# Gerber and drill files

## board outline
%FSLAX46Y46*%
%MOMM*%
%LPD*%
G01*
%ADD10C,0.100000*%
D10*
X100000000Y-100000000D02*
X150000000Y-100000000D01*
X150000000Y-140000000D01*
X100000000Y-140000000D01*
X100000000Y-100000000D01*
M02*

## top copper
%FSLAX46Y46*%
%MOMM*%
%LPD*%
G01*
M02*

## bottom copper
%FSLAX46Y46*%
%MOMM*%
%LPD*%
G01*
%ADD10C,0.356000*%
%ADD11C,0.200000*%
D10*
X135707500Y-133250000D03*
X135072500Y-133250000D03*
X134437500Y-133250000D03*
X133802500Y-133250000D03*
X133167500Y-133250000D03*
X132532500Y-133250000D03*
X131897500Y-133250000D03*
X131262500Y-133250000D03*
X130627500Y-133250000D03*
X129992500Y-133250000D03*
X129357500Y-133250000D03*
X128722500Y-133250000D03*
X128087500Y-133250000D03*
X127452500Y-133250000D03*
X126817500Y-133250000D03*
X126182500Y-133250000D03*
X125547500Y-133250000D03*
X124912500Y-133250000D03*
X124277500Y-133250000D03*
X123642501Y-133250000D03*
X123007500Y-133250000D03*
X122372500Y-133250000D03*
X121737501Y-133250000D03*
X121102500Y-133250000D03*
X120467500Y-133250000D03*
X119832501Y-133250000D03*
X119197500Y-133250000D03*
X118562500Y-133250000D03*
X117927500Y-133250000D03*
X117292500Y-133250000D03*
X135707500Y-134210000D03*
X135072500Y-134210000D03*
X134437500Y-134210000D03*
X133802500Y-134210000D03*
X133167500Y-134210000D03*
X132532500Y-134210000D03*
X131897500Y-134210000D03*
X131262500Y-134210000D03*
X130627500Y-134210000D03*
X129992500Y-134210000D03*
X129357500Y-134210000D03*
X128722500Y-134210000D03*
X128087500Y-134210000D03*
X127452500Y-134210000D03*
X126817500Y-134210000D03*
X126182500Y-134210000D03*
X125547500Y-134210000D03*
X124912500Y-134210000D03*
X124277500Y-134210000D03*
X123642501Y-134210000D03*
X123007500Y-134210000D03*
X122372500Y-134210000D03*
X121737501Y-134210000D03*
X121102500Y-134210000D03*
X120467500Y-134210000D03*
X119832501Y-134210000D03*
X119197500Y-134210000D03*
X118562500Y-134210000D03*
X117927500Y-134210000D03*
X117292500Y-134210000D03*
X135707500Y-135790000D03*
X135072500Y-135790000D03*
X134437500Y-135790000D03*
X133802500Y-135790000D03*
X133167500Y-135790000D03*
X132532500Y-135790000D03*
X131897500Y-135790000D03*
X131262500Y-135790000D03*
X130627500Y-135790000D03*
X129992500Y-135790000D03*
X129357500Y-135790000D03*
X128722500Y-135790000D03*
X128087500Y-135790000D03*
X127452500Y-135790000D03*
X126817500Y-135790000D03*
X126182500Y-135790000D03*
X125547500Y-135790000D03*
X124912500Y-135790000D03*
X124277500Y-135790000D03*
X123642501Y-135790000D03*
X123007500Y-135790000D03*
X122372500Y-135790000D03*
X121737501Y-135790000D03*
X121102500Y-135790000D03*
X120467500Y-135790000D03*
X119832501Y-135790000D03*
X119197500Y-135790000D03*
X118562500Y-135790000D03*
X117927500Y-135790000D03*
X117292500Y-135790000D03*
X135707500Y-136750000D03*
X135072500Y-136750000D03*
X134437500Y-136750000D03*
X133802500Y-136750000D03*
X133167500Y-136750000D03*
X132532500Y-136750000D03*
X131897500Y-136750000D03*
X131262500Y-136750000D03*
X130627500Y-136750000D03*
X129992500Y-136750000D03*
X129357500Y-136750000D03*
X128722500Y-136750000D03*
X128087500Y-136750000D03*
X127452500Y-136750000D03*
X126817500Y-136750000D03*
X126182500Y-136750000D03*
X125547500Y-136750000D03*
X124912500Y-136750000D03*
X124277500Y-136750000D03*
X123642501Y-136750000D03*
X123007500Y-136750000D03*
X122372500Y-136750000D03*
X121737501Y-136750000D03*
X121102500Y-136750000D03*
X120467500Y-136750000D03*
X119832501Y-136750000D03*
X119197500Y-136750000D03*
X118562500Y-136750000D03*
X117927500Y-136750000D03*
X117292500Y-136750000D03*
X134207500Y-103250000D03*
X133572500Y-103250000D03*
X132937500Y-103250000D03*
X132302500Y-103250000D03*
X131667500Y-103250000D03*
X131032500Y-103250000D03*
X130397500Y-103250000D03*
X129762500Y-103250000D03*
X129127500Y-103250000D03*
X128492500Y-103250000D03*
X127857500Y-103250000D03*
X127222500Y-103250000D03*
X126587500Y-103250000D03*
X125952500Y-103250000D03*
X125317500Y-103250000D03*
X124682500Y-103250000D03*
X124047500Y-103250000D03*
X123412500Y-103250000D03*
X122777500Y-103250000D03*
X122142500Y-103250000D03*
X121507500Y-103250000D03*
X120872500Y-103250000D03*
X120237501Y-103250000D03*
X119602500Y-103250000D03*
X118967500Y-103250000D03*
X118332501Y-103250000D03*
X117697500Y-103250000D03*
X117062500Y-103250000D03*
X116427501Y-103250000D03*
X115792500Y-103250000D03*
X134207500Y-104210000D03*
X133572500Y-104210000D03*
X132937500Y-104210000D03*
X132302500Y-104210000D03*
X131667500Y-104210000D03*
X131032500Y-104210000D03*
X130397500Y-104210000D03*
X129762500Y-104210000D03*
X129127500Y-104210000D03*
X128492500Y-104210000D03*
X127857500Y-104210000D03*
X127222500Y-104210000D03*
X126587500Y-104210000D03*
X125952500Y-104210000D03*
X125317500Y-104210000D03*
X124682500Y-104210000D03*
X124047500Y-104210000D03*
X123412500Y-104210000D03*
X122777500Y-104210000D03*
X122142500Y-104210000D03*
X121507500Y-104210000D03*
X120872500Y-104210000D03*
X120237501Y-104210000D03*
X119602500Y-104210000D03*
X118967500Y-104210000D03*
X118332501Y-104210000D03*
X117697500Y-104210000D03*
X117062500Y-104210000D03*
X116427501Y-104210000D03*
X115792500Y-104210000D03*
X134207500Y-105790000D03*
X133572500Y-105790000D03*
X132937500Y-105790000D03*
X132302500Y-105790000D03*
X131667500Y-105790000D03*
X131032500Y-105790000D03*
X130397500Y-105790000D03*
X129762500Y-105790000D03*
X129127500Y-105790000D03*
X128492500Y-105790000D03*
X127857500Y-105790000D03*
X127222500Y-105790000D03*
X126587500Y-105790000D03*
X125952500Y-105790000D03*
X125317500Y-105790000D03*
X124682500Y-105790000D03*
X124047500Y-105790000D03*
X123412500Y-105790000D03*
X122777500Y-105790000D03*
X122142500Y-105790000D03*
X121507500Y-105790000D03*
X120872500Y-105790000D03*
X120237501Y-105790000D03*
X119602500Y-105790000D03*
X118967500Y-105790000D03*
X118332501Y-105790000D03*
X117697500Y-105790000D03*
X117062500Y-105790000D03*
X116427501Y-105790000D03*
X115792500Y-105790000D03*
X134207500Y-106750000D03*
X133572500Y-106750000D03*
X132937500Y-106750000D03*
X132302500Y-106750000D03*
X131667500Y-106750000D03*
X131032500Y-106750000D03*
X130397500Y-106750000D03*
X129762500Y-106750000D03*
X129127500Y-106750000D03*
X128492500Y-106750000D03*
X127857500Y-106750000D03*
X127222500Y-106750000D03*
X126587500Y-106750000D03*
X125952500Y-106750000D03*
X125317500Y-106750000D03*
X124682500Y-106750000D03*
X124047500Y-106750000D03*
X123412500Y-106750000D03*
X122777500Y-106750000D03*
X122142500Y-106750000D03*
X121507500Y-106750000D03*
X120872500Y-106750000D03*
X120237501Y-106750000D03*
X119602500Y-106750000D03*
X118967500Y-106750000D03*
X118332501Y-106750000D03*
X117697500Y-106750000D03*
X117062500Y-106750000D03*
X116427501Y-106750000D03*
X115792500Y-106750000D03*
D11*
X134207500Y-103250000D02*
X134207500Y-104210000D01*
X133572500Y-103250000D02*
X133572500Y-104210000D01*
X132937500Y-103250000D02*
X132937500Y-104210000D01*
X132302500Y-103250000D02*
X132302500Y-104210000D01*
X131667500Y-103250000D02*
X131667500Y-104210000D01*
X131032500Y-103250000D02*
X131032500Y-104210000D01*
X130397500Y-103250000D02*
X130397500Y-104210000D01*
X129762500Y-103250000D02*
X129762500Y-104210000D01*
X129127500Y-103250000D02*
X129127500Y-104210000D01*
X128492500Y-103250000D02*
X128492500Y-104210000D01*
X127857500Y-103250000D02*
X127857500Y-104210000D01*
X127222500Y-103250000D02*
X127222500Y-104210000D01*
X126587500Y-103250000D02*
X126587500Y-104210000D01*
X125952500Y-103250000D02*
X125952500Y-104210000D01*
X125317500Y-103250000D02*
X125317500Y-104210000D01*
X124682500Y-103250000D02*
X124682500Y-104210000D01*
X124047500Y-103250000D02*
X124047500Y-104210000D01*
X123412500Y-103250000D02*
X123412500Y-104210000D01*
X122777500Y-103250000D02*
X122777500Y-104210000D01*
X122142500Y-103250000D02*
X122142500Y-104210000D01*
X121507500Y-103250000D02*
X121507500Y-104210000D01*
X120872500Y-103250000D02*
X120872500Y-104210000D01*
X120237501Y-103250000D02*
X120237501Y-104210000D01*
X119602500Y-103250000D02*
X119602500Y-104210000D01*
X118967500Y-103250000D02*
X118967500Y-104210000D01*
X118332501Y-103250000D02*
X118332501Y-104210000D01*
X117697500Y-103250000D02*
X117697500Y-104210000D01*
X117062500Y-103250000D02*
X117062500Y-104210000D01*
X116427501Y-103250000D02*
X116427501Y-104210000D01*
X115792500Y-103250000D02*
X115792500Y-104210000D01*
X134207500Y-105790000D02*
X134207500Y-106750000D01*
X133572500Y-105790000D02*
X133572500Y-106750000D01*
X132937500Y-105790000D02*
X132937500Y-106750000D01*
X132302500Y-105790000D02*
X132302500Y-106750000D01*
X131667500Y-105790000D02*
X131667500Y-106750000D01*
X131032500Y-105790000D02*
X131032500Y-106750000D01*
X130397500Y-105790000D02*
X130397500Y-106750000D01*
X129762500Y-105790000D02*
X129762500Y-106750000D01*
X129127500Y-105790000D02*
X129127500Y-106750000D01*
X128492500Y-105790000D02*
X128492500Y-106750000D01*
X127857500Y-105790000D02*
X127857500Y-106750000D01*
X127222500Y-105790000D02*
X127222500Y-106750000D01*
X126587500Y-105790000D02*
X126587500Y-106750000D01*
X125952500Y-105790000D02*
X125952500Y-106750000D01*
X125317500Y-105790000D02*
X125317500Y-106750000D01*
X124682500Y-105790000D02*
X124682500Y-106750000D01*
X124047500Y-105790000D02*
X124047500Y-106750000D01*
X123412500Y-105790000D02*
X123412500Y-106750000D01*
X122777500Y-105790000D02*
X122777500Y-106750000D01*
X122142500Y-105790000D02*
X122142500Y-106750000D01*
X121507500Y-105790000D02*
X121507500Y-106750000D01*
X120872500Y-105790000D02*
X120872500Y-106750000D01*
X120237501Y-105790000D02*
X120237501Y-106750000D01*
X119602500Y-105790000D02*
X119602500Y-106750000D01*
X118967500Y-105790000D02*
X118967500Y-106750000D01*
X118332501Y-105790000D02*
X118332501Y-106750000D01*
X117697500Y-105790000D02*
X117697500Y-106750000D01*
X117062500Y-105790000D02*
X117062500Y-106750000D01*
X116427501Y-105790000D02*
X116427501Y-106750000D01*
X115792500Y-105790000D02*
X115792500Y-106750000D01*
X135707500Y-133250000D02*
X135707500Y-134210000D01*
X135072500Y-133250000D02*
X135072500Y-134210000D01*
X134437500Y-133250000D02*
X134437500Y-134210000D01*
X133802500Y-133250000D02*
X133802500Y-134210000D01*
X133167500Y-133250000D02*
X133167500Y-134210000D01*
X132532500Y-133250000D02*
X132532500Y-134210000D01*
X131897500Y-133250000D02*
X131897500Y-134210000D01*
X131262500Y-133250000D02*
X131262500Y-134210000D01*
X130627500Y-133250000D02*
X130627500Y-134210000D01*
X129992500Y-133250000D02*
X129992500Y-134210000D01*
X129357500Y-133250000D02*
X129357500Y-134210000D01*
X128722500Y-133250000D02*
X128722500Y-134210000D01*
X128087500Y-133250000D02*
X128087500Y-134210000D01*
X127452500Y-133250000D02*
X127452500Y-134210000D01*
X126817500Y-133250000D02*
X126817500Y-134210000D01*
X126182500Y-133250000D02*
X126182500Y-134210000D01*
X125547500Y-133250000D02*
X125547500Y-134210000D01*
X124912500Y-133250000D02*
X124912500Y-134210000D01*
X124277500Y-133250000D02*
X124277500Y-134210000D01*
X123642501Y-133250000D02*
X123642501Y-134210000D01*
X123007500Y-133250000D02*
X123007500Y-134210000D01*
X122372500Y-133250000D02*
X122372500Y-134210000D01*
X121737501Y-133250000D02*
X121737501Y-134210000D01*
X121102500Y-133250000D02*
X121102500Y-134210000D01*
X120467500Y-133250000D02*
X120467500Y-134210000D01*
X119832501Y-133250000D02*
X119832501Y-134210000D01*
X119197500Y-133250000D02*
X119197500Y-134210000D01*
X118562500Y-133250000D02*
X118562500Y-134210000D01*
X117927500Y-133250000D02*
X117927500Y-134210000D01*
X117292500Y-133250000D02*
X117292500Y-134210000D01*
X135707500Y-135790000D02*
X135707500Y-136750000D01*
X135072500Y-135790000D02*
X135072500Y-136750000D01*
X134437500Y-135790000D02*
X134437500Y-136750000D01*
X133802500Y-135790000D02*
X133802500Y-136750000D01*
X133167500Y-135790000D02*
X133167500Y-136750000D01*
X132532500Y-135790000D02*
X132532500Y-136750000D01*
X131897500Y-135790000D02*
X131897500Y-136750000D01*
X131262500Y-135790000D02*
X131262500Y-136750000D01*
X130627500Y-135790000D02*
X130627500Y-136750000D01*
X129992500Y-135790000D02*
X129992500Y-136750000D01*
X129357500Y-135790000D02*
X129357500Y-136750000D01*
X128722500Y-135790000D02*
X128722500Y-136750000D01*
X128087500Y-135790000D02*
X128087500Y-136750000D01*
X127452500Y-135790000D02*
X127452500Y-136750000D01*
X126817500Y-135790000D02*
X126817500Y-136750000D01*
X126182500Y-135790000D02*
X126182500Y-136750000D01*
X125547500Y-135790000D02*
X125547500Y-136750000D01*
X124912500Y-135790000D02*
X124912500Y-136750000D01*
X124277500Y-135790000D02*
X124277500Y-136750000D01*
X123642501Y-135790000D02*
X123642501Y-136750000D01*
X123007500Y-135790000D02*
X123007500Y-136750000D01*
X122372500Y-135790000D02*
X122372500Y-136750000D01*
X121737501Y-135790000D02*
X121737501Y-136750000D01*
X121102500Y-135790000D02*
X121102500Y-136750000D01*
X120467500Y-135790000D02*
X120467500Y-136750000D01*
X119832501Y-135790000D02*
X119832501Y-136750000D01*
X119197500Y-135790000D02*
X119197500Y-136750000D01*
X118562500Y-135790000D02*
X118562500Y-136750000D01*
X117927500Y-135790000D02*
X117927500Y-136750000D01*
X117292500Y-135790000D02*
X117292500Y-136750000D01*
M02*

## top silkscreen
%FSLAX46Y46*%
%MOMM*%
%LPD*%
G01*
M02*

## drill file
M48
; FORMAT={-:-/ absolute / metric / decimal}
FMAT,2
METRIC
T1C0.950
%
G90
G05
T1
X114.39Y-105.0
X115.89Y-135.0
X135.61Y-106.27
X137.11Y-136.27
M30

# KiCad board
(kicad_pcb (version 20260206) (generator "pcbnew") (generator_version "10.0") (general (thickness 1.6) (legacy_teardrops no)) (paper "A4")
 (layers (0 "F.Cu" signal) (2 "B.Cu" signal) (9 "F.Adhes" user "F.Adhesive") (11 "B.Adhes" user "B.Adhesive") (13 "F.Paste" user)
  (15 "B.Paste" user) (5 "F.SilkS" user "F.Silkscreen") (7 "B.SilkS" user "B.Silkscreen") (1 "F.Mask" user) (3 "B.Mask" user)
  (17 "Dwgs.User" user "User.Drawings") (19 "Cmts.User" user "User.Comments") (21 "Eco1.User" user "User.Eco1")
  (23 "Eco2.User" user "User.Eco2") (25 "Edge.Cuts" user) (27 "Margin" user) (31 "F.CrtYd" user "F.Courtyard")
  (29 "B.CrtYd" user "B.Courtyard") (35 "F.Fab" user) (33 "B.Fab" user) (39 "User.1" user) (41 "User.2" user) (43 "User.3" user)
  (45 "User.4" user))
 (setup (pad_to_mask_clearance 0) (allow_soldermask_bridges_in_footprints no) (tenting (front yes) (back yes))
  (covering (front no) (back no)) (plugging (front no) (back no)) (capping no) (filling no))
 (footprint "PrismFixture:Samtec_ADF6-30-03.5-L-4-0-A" (layer "B.Cu") (at 126.5 135)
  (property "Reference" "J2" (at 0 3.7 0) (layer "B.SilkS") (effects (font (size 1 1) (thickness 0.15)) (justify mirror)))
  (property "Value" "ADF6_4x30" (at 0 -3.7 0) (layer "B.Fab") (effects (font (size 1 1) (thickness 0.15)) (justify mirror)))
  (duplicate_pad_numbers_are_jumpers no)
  (pad "" np_thru_hole circle (at -10.61 0) (size 0.95 0.95) (drill 0.95) (layers "*.Cu" "*.Mask"))
  (pad "" np_thru_hole circle (at 10.61 1.27) (size 0.95 0.95) (drill 0.95) (layers "*.Cu" "*.Mask"))
  (pad "A01" smd circle (at 9.2075 -1.75) (size 0.356 0.356) (layers "B.Cu" "B.Mask" "B.Paste") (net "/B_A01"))
  (pad "A02" smd circle (at 8.5725 -1.75) (size 0.356 0.356) (layers "B.Cu" "B.Mask" "B.Paste") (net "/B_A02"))
  (pad "A03" smd circle (at 7.9375 -1.75) (size 0.356 0.356) (layers "B.Cu" "B.Mask" "B.Paste") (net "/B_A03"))
  (pad "A04" smd circle (at 7.3025 -1.75) (size 0.356 0.356) (layers "B.Cu" "B.Mask" "B.Paste") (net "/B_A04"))
  (pad "A05" smd circle (at 6.6675 -1.75) (size 0.356 0.356) (layers "B.Cu" "B.Mask" "B.Paste") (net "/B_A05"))
  (pad "A06" smd circle (at 6.0325 -1.75) (size 0.356 0.356) (layers "B.Cu" "B.Mask" "B.Paste") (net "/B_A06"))
  (pad "A07" smd circle (at 5.3975 -1.75) (size 0.356 0.356) (layers "B.Cu" "B.Mask" "B.Paste") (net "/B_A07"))
  (pad "A08" smd circle (at 4.7625 -1.75) (size 0.356 0.356) (layers "B.Cu" "B.Mask" "B.Paste") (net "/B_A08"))
  (pad "A09" smd circle (at 4.1275 -1.75) (size 0.356 0.356) (layers "B.Cu" "B.Mask" "B.Paste") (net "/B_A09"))
  (pad "A10" smd circle (at 3.4925 -1.75) (size 0.356 0.356) (layers "B.Cu" "B.Mask" "B.Paste") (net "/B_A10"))
  (pad "A11" smd circle (at 2.8575 -1.75) (size 0.356 0.356) (layers "B.Cu" "B.Mask" "B.Paste") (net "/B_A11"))
  (pad "A12" smd circle (at 2.2225 -1.75) (size 0.356 0.356) (layers "B.Cu" "B.Mask" "B.Paste") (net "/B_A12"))
  (pad "A13" smd circle (at 1.5875 -1.75) (size 0.356 0.356) (layers "B.Cu" "B.Mask" "B.Paste") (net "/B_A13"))
  (pad "A14" smd circle (at 0.9525 -1.75) (size 0.356 0.356) (layers "B.Cu" "B.Mask" "B.Paste") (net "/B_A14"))
  (pad "A15" smd circle (at 0.3175 -1.75) (size 0.356 0.356) (layers "B.Cu" "B.Mask" "B.Paste") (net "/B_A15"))
  (pad "A16" smd circle (at -0.3175 -1.75) (size 0.356 0.356) (layers "B.Cu" "B.Mask" "B.Paste") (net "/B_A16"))
  (pad "A17" smd circle (at -0.9525 -1.75) (size 0.356 0.356) (layers "B.Cu" "B.Mask" "B.Paste") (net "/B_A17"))
  (pad "A18" smd circle (at -1.5875 -1.75) (size 0.356 0.356) (layers "B.Cu" "B.Mask" "B.Paste") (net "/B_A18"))
  (pad "A19" smd circle (at -2.2225 -1.75) (size 0.356 0.356) (layers "B.Cu" "B.Mask" "B.Paste") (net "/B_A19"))
  (pad "A20" smd circle (at -2.857499 -1.75) (size 0.356 0.356) (layers "B.Cu" "B.Mask" "B.Paste") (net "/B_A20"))
  (pad "A21" smd circle (at -3.4925 -1.75) (size 0.356 0.356) (layers "B.Cu" "B.Mask" "B.Paste") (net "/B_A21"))
  (pad "A22" smd circle (at -4.1275 -1.75) (size 0.356 0.356) (layers "B.Cu" "B.Mask" "B.Paste") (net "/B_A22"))
  (pad "A23" smd circle (at -4.762499 -1.75) (size 0.356 0.356) (layers "B.Cu" "B.Mask" "B.Paste") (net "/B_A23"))
  (pad "A24" smd circle (at -5.3975 -1.75) (size 0.356 0.356) (layers "B.Cu" "B.Mask" "B.Paste") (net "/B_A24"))
  (pad "A25" smd circle (at -6.0325 -1.75) (size 0.356 0.356) (layers "B.Cu" "B.Mask" "B.Paste") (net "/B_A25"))
  (pad "A26" smd circle (at -6.667499 -1.75) (size 0.356 0.356) (layers "B.Cu" "B.Mask" "B.Paste") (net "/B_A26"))
  (pad "A27" smd circle (at -7.3025 -1.75) (size 0.356 0.356) (layers "B.Cu" "B.Mask" "B.Paste") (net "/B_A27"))
  (pad "A28" smd circle (at -7.9375 -1.75) (size 0.356 0.356) (layers "B.Cu" "B.Mask" "B.Paste") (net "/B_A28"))
  (pad "A29" smd circle (at -8.5725 -1.75) (size 0.356 0.356) (layers "B.Cu" "B.Mask" "B.Paste") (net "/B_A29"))
  (pad "A30" smd circle (at -9.2075 -1.75) (size 0.356 0.356) (layers "B.Cu" "B.Mask" "B.Paste") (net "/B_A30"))
  (pad "B01" smd circle (at 9.2075 -0.79) (size 0.356 0.356) (layers "B.Cu" "B.Mask" "B.Paste") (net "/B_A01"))
  (pad "B02" smd circle (at 8.5725 -0.79) (size 0.356 0.356) (layers "B.Cu" "B.Mask" "B.Paste") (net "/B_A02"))
  (pad "B03" smd circle (at 7.9375 -0.79) (size 0.356 0.356) (layers "B.Cu" "B.Mask" "B.Paste") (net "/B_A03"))
  (pad "B04" smd circle (at 7.3025 -0.79) (size 0.356 0.356) (layers "B.Cu" "B.Mask" "B.Paste") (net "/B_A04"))
  (pad "B05" smd circle (at 6.6675 -0.79) (size 0.356 0.356) (layers "B.Cu" "B.Mask" "B.Paste") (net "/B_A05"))
  (pad "B06" smd circle (at 6.0325 -0.79) (size 0.356 0.356) (layers "B.Cu" "B.Mask" "B.Paste") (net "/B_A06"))
  (pad "B07" smd circle (at 5.3975 -0.79) (size 0.356 0.356) (layers "B.Cu" "B.Mask" "B.Paste") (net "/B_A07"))
  (pad "B08" smd circle (at 4.7625 -0.79) (size 0.356 0.356) (layers "B.Cu" "B.Mask" "B.Paste") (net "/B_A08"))
  (pad "B09" smd circle (at 4.1275 -0.79) (size 0.356 0.356) (layers "B.Cu" "B.Mask" "B.Paste") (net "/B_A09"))
  (pad "B10" smd circle (at 3.4925 -0.79) (size 0.356 0.356) (layers "B.Cu" "B.Mask" "B.Paste") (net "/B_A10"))
  (pad "B11" smd circle (at 2.8575 -0.79) (size 0.356 0.356) (layers "B.Cu" "B.Mask" "B.Paste") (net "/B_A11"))
  (pad "B12" smd circle (at 2.2225 -0.79) (size 0.356 0.356) (layers "B.Cu" "B.Mask" "B.Paste") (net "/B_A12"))
  (pad "B13" smd circle (at 1.5875 -0.79) (size 0.356 0.356) (layers "B.Cu" "B.Mask" "B.Paste") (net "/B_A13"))
  (pad "B14" smd circle (at 0.9525 -0.79) (size 0.356 0.356) (layers "B.Cu" "B.Mask" "B.Paste") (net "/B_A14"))
  (pad "B15" smd circle (at 0.3175 -0.79) (size 0.356 0.356) (layers "B.Cu" "B.Mask" "B.Paste") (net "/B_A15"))
  (pad "B16" smd circle (at -0.3175 -0.79) (size 0.356 0.356) (layers "B.Cu" "B.Mask" "B.Paste") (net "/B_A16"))
  (pad "B17" smd circle (at -0.9525 -0.79) (size 0.356 0.356) (layers "B.Cu" "B.Mask" "B.Paste") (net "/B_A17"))
  (pad "B18" smd circle (at -1.5875 -0.79) (size 0.356 0.356) (layers "B.Cu" "B.Mask" "B.Paste") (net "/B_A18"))
  (pad "B19" smd circle (at -2.2225 -0.79) (size 0.356 0.356) (layers "B.Cu" "B.Mask" "B.Paste") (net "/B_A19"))
  (pad "B20" smd circle (at -2.857499 -0.79) (size 0.356 0.356) (layers "B.Cu" "B.Mask" "B.Paste") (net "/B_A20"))
  (pad "B21" smd circle (at -3.4925 -0.79) (size 0.356 0.356) (layers "B.Cu" "B.Mask" "B.Paste") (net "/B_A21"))
  (pad "B22" smd circle (at -4.1275 -0.79) (size 0.356 0.356) (layers "B.Cu" "B.Mask" "B.Paste") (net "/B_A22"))
  (pad "B23" smd circle (at -4.762499 -0.79) (size 0.356 0.356) (layers "B.Cu" "B.Mask" "B.Paste") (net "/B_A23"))
  (pad "B24" smd circle (at -5.3975 -0.79) (size 0.356 0.356) (layers "B.Cu" "B.Mask" "B.Paste") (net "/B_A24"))
  (pad "B25" smd circle (at -6.0325 -0.79) (size 0.356 0.356) (layers "B.Cu" "B.Mask" "B.Paste") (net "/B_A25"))
  (pad "B26" smd circle (at -6.667499 -0.79) (size 0.356 0.356) (layers "B.Cu" "B.Mask" "B.Paste") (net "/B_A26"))
  (pad "B27" smd circle (at -7.3025 -0.79) (size 0.356 0.356) (layers "B.Cu" "B.Mask" "B.Paste") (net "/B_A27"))
  (pad "B28" smd circle (at -7.9375 -0.79) (size 0.356 0.356) (layers "B.Cu" "B.Mask" "B.Paste") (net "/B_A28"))
  (pad "B29" smd circle (at -8.5725 -0.79) (size 0.356 0.356) (layers "B.Cu" "B.Mask" "B.Paste") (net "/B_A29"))
  (pad "B30" smd circle (at -9.2075 -0.79) (size 0.356 0.356) (layers "B.Cu" "B.Mask" "B.Paste") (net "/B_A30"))
  (pad "C01" smd circle (at 9.2075 0.79) (size 0.356 0.356) (layers "B.Cu" "B.Mask" "B.Paste") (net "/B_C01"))
  (pad "C02" smd circle (at 8.5725 0.79) (size 0.356 0.356) (layers "B.Cu" "B.Mask" "B.Paste") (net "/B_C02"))
  (pad "C03" smd circle (at 7.9375 0.79) (size 0.356 0.356) (layers "B.Cu" "B.Mask" "B.Paste") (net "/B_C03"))
  (pad "C04" smd circle (at 7.3025 0.79) (size 0.356 0.356) (layers "B.Cu" "B.Mask" "B.Paste") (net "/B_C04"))
  (pad "C05" smd circle (at 6.6675 0.79) (size 0.356 0.356) (layers "B.Cu" "B.Mask" "B.Paste") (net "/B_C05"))
  (pad "C06" smd circle (at 6.0325 0.79) (size 0.356 0.356) (layers "B.Cu" "B.Mask" "B.Paste") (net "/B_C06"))
  (pad "C07" smd circle (at 5.3975 0.79) (size 0.356 0.356) (layers "B.Cu" "B.Mask" "B.Paste") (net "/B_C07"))
  (pad "C08" smd circle (at 4.7625 0.79) (size 0.356 0.356) (layers "B.Cu" "B.Mask" "B.Paste") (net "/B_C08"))
  (pad "C09" smd circle (at 4.1275 0.79) (size 0.356 0.356) (layers "B.Cu" "B.Mask" "B.Paste") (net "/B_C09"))
  (pad "C10" smd circle (at 3.4925 0.79) (size 0.356 0.356) (layers "B.Cu" "B.Mask" "B.Paste") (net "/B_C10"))
  (pad "C11" smd circle (at 2.8575 0.79) (size 0.356 0.356) (layers "B.Cu" "B.Mask" "B.Paste") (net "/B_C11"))
  (pad "C12" smd circle (at 2.2225 0.79) (size 0.356 0.356) (layers "B.Cu" "B.Mask" "B.Paste") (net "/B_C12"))
  (pad "C13" smd circle (at 1.5875 0.79) (size 0.356 0.356) (layers "B.Cu" "B.Mask" "B.Paste") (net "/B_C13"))
  (pad "C14" smd circle (at 0.9525 0.79) (size 0.356 0.356) (layers "B.Cu" "B.Mask" "B.Paste") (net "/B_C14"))
  (pad "C15" smd circle (at 0.3175 0.79) (size 0.356 0.356) (layers "B.Cu" "B.Mask" "B.Paste") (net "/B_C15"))
  (pad "C16" smd circle (at -0.3175 0.79) (size 0.356 0.356) (layers "B.Cu" "B.Mask" "B.Paste") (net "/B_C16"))
  (pad "C17" smd circle (at -0.9525 0.79) (size 0.356 0.356) (layers "B.Cu" "B.Mask" "B.Paste") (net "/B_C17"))
  (pad "C18" smd circle (at -1.5875 0.79) (size 0.356 0.356) (layers "B.Cu" "B.Mask" "B.Paste") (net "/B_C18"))
  (pad "C19" smd circle (at -2.2225 0.79) (size 0.356 0.356) (layers "B.Cu" "B.Mask" "B.Paste") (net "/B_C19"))
  (pad "C20" smd circle (at -2.857499 0.79) (size 0.356 0.356) (layers "B.Cu" "B.Mask" "B.Paste") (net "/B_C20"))
  (pad "C21" smd circle (at -3.4925 0.79) (size 0.356 0.356) (layers "B.Cu" "B.Mask" "B.Paste") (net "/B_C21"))
  (pad "C22" smd circle (at -4.1275 0.79) (size 0.356 0.356) (layers "B.Cu" "B.Mask" "B.Paste") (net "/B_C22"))
  (pad "C23" smd circle (at -4.762499 0.79) (size 0.356 0.356) (layers "B.Cu" "B.Mask" "B.Paste") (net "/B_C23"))
  (pad "C24" smd circle (at -5.3975 0.79) (size 0.356 0.356) (layers "B.Cu" "B.Mask" "B.Paste") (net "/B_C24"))
  (pad "C25" smd circle (at -6.0325 0.79) (size 0.356 0.356) (layers "B.Cu" "B.Mask" "B.Paste") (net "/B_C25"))
  (pad "C26" smd circle (at -6.667499 0.79) (size 0.356 0.356) (layers "B.Cu" "B.Mask" "B.Paste") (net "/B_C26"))
  (pad "C27" smd circle (at -7.3025 0.79) (size 0.356 0.356) (layers "B.Cu" "B.Mask" "B.Paste") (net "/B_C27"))
  (pad "C28" smd circle (at -7.9375 0.79) (size 0.356 0.356) (layers "B.Cu" "B.Mask" "B.Paste") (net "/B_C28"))
  (pad "C29" smd circle (at -8.5725 0.79) (size 0.356 0.356) (layers "B.Cu" "B.Mask" "B.Paste") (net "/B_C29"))
  (pad "C30" smd circle (at -9.2075 0.79) (size 0.356 0.356) (layers "B.Cu" "B.Mask" "B.Paste") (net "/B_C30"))
  (pad "D01" smd circle (at 9.2075 1.75) (size 0.356 0.356) (layers "B.Cu" "B.Mask" "B.Paste") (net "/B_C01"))
  (pad "D02" smd circle (at 8.5725 1.75) (size 0.356 0.356) (layers "B.Cu" "B.Mask" "B.Paste") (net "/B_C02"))
  (pad "D03" smd circle (at 7.9375 1.75) (size 0.356 0.356) (layers "B.Cu" "B.Mask" "B.Paste") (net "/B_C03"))
  (pad "D04" smd circle (at 7.3025 1.75) (size 0.356 0.356) (layers "B.Cu" "B.Mask" "B.Paste") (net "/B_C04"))
  (pad "D05" smd circle (at 6.6675 1.75) (size 0.356 0.356) (layers "B.Cu" "B.Mask" "B.Paste") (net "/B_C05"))
  (pad "D06" smd circle (at 6.0325 1.75) (size 0.356 0.356) (layers "B.Cu" "B.Mask" "B.Paste") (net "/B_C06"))
  (pad "D07" smd circle (at 5.3975 1.75) (size 0.356 0.356) (layers "B.Cu" "B.Mask" "B.Paste") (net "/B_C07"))
  (pad "D08" smd circle (at 4.7625 1.75) (size 0.356 0.356) (layers "B.Cu" "B.Mask" "B.Paste") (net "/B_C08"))
  (pad "D09" smd circle (at 4.1275 1.75) (size 0.356 0.356) (layers "B.Cu" "B.Mask" "B.Paste") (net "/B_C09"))
  (pad "D10" smd circle (at 3.4925 1.75) (size 0.356 0.356) (layers "B.Cu" "B.Mask" "B.Paste") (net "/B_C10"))
  (pad "D11" smd circle (at 2.8575 1.75) (size 0.356 0.356) (layers "B.Cu" "B.Mask" "B.Paste") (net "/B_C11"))
  (pad "D12" smd circle (at 2.2225 1.75) (size 0.356 0.356) (layers "B.Cu" "B.Mask" "B.Paste") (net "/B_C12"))
  (pad "D13" smd circle (at 1.5875 1.75) (size 0.356 0.356) (layers "B.Cu" "B.Mask" "B.Paste") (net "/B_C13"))
  (pad "D14" smd circle (at 0.9525 1.75) (size 0.356 0.356) (layers "B.Cu" "B.Mask" "B.Paste") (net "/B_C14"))
  (pad "D15" smd circle (at 0.3175 1.75) (size 0.356 0.356) (layers "B.Cu" "B.Mask" "B.Paste") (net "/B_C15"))
  (pad "D16" smd circle (at -0.3175 1.75) (size 0.356 0.356) (layers "B.Cu" "B.Mask" "B.Paste") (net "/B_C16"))
  (pad "D17" smd circle (at -0.9525 1.75) (size 0.356 0.356) (layers "B.Cu" "B.Mask" "B.Paste") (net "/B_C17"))
  (pad "D18" smd circle (at -1.5875 1.75) (size 0.356 0.356) (layers "B.Cu" "B.Mask" "B.Paste") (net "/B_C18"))
  (pad "D19" smd circle (at -2.2225 1.75) (size 0.356 0.356) (layers "B.Cu" "B.Mask" "B.Paste") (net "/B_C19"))
  (pad "D20" smd circle (at -2.857499 1.75) (size 0.356 0.356) (layers "B.Cu" "B.Mask" "B.Paste") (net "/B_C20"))
  (pad "D21" smd circle (at -3.4925 1.75) (size 0.356 0.356) (layers "B.Cu" "B.Mask" "B.Paste") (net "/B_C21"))
  (pad "D22" smd circle (at -4.1275 1.75) (size 0.356 0.356) (layers "B.Cu" "B.Mask" "B.Paste") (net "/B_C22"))
  (pad "D23" smd circle (at -4.762499 1.75) (size 0.356 0.356) (layers "B.Cu" "B.Mask" "B.Paste") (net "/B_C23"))
  (pad "D24" smd circle (at -5.3975 1.75) (size 0.356 0.356) (layers "B.Cu" "B.Mask" "B.Paste") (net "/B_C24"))
  (pad "D25" smd circle (at -6.0325 1.75) (size 0.356 0.356) (layers "B.Cu" "B.Mask" "B.Paste") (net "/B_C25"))
  (pad "D26" smd circle (at -6.667499 1.75) (size 0.356 0.356) (layers "B.Cu" "B.Mask" "B.Paste") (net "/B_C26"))
  (pad "D27" smd circle (at -7.3025 1.75) (size 0.356 0.356) (layers "B.Cu" "B.Mask" "B.Paste") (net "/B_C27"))
  (pad "D28" smd circle (at -7.9375 1.75) (size 0.356 0.356) (layers "B.Cu" "B.Mask" "B.Paste") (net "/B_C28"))
  (pad "D29" smd circle (at -8.5725 1.75) (size 0.356 0.356) (layers "B.Cu" "B.Mask" "B.Paste") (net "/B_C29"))
  (pad "D30" smd circle (at -9.2075 1.75) (size 0.356 0.356) (layers "B.Cu" "B.Mask" "B.Paste") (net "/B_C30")))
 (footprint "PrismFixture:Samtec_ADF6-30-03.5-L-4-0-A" (layer "B.Cu") (at 125 105)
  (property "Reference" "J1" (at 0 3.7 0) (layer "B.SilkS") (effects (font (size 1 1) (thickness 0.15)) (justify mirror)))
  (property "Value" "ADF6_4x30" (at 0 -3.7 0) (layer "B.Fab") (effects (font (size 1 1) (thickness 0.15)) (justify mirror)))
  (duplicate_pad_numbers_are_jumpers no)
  (pad "" np_thru_hole circle (at -10.61 0) (size 0.95 0.95) (drill 0.95) (layers "*.Cu" "*.Mask"))
  (pad "" np_thru_hole circle (at 10.61 1.27) (size 0.95 0.95) (drill 0.95) (layers "*.Cu" "*.Mask"))
  (pad "A01" smd circle (at 9.2075 -1.75) (size 0.356 0.356) (layers "B.Cu" "B.Mask" "B.Paste") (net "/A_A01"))
  (pad "A02" smd circle (at 8.5725 -1.75) (size 0.356 0.356) (layers "B.Cu" "B.Mask" "B.Paste") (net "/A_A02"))
  (pad "A03" smd circle (at 7.9375 -1.75) (size 0.356 0.356) (layers "B.Cu" "B.Mask" "B.Paste") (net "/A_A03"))
  (pad "A04" smd circle (at 7.3025 -1.75) (size 0.356 0.356) (layers "B.Cu" "B.Mask" "B.Paste") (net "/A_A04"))
  (pad "A05" smd circle (at 6.6675 -1.75) (size 0.356 0.356) (layers "B.Cu" "B.Mask" "B.Paste") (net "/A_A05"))
  (pad "A06" smd circle (at 6.0325 -1.75) (size 0.356 0.356) (layers "B.Cu" "B.Mask" "B.Paste") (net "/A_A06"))
  (pad "A07" smd circle (at 5.3975 -1.75) (size 0.356 0.356) (layers "B.Cu" "B.Mask" "B.Paste") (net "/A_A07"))
  (pad "A08" smd circle (at 4.7625 -1.75) (size 0.356 0.356) (layers "B.Cu" "B.Mask" "B.Paste") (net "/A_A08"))
  (pad "A09" smd circle (at 4.1275 -1.75) (size 0.356 0.356) (layers "B.Cu" "B.Mask" "B.Paste") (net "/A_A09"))
  (pad "A10" smd circle (at 3.4925 -1.75) (size 0.356 0.356) (layers "B.Cu" "B.Mask" "B.Paste") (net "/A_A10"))
  (pad "A11" smd circle (at 2.8575 -1.75) (size 0.356 0.356) (layers "B.Cu" "B.Mask" "B.Paste") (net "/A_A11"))
  (pad "A12" smd circle (at 2.2225 -1.75) (size 0.356 0.356) (layers "B.Cu" "B.Mask" "B.Paste") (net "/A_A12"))
  (pad "A13" smd circle (at 1.5875 -1.75) (size 0.356 0.356) (layers "B.Cu" "B.Mask" "B.Paste") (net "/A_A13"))
  (pad "A14" smd circle (at 0.9525 -1.75) (size 0.356 0.356) (layers "B.Cu" "B.Mask" "B.Paste") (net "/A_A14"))
  (pad "A15" smd circle (at 0.3175 -1.75) (size 0.356 0.356) (layers "B.Cu" "B.Mask" "B.Paste") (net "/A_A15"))
  (pad "A16" smd circle (at -0.3175 -1.75) (size 0.356 0.356) (layers "B.Cu" "B.Mask" "B.Paste") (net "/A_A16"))
  (pad "A17" smd circle (at -0.9525 -1.75) (size 0.356 0.356) (layers "B.Cu" "B.Mask" "B.Paste") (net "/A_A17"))
  (pad "A18" smd circle (at -1.5875 -1.75) (size 0.356 0.356) (layers "B.Cu" "B.Mask" "B.Paste") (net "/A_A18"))
  (pad "A19" smd circle (at -2.2225 -1.75) (size 0.356 0.356) (layers "B.Cu" "B.Mask" "B.Paste") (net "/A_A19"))
  (pad "A20" smd circle (at -2.8575 -1.75) (size 0.356 0.356) (layers "B.Cu" "B.Mask" "B.Paste") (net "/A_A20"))
  (pad "A21" smd circle (at -3.4925 -1.75) (size 0.356 0.356) (layers "B.Cu" "B.Mask" "B.Paste") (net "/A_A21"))
  (pad "A22" smd circle (at -4.1275 -1.75) (size 0.356 0.356) (layers "B.Cu" "B.Mask" "B.Paste") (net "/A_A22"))
  (pad "A23" smd circle (at -4.762499 -1.75) (size 0.356 0.356) (layers "B.Cu" "B.Mask" "B.Paste") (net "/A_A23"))
  (pad "A24" smd circle (at -5.3975 -1.75) (size 0.356 0.356) (layers "B.Cu" "B.Mask" "B.Paste") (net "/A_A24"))
  (pad "A25" smd circle (at -6.0325 -1.75) (size 0.356 0.356) (layers "B.Cu" "B.Mask" "B.Paste") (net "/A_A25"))
  (pad "A26" smd circle (at -6.667499 -1.75) (size 0.356 0.356) (layers "B.Cu" "B.Mask" "B.Paste") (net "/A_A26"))
  (pad "A27" smd circle (at -7.3025 -1.75) (size 0.356 0.356) (layers "B.Cu" "B.Mask" "B.Paste") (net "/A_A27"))
  (pad "A28" smd circle (at -7.9375 -1.75) (size 0.356 0.356) (layers "B.Cu" "B.Mask" "B.Paste") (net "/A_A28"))
  (pad "A29" smd circle (at -8.572499 -1.75) (size 0.356 0.356) (layers "B.Cu" "B.Mask" "B.Paste") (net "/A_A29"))
  (pad "A30" smd circle (at -9.2075 -1.75) (size 0.356 0.356) (layers "B.Cu" "B.Mask" "B.Paste") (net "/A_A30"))
  (pad "B01" smd circle (at 9.2075 -0.79) (size 0.356 0.356) (layers "B.Cu" "B.Mask" "B.Paste") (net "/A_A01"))
  (pad "B02" smd circle (at 8.5725 -0.79) (size 0.356 0.356) (layers "B.Cu" "B.Mask" "B.Paste") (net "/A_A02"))
  (pad "B03" smd circle (at 7.9375 -0.79) (size 0.356 0.356) (layers "B.Cu" "B.Mask" "B.Paste") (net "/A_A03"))
  (pad "B04" smd circle (at 7.3025 -0.79) (size 0.356 0.356) (layers "B.Cu" "B.Mask" "B.Paste") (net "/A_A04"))
  (pad "B05" smd circle (at 6.6675 -0.79) (size 0.356 0.356) (layers "B.Cu" "B.Mask" "B.Paste") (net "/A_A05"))
  (pad "B06" smd circle (at 6.0325 -0.79) (size 0.356 0.356) (layers "B.Cu" "B.Mask" "B.Paste") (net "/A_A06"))
  (pad "B07" smd circle (at 5.3975 -0.79) (size 0.356 0.356) (layers "B.Cu" "B.Mask" "B.Paste") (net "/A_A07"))
  (pad "B08" smd circle (at 4.7625 -0.79) (size 0.356 0.356) (layers "B.Cu" "B.Mask" "B.Paste") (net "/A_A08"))
  (pad "B09" smd circle (at 4.1275 -0.79) (size 0.356 0.356) (layers "B.Cu" "B.Mask" "B.Paste") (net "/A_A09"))
  (pad "B10" smd circle (at 3.4925 -0.79) (size 0.356 0.356) (layers "B.Cu" "B.Mask" "B.Paste") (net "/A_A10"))
  (pad "B11" smd circle (at 2.8575 -0.79) (size 0.356 0.356) (layers "B.Cu" "B.Mask" "B.Paste") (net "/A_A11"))
  (pad "B12" smd circle (at 2.2225 -0.79) (size 0.356 0.356) (layers "B.Cu" "B.Mask" "B.Paste") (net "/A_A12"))
  (pad "B13" smd circle (at 1.5875 -0.79) (size 0.356 0.356) (layers "B.Cu" "B.Mask" "B.Paste") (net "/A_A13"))
  (pad "B14" smd circle (at 0.9525 -0.79) (size 0.356 0.356) (layers "B.Cu" "B.Mask" "B.Paste") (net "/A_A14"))
  (pad "B15" smd circle (at 0.3175 -0.79) (size 0.356 0.356) (layers "B.Cu" "B.Mask" "B.Paste") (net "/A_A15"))
  (pad "B16" smd circle (at -0.3175 -0.79) (size 0.356 0.356) (layers "B.Cu" "B.Mask" "B.Paste") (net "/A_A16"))
  (pad "B17" smd circle (at -0.9525 -0.79) (size 0.356 0.356) (layers "B.Cu" "B.Mask" "B.Paste") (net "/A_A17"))
  (pad "B18" smd circle (at -1.5875 -0.79) (size 0.356 0.356) (layers "B.Cu" "B.Mask" "B.Paste") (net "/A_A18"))
  (pad "B19" smd circle (at -2.2225 -0.79) (size 0.356 0.356) (layers "B.Cu" "B.Mask" "B.Paste") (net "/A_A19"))
  (pad "B20" smd circle (at -2.8575 -0.79) (size 0.356 0.356) (layers "B.Cu" "B.Mask" "B.Paste") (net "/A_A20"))
  (pad "B21" smd circle (at -3.4925 -0.79) (size 0.356 0.356) (layers "B.Cu" "B.Mask" "B.Paste") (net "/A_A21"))
  (pad "B22" smd circle (at -4.1275 -0.79) (size 0.356 0.356) (layers "B.Cu" "B.Mask" "B.Paste") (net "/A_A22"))
  (pad "B23" smd circle (at -4.762499 -0.79) (size 0.356 0.356) (layers "B.Cu" "B.Mask" "B.Paste") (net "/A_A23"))
  (pad "B24" smd circle (at -5.3975 -0.79) (size 0.356 0.356) (layers "B.Cu" "B.Mask" "B.Paste") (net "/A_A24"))
  (pad "B25" smd circle (at -6.0325 -0.79) (size 0.356 0.356) (layers "B.Cu" "B.Mask" "B.Paste") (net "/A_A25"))
  (pad "B26" smd circle (at -6.667499 -0.79) (size 0.356 0.356) (layers "B.Cu" "B.Mask" "B.Paste") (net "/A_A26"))
  (pad "B27" smd circle (at -7.3025 -0.79) (size 0.356 0.356) (layers "B.Cu" "B.Mask" "B.Paste") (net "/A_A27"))
  (pad "B28" smd circle (at -7.9375 -0.79) (size 0.356 0.356) (layers "B.Cu" "B.Mask" "B.Paste") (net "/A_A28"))
  (pad "B29" smd circle (at -8.572499 -0.79) (size 0.356 0.356) (layers "B.Cu" "B.Mask" "B.Paste") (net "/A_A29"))
  (pad "B30" smd circle (at -9.2075 -0.79) (size 0.356 0.356) (layers "B.Cu" "B.Mask" "B.Paste") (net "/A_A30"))
  (pad "C01" smd circle (at 9.2075 0.79) (size 0.356 0.356) (layers "B.Cu" "B.Mask" "B.Paste") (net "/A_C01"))
  (pad "C02" smd circle (at 8.5725 0.79) (size 0.356 0.356) (layers "B.Cu" "B.Mask" "B.Paste") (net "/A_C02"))
  (pad "C03" smd circle (at 7.9375 0.79) (size 0.356 0.356) (layers "B.Cu" "B.Mask" "B.Paste") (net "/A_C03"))
  (pad "C04" smd circle (at 7.3025 0.79) (size 0.356 0.356) (layers "B.Cu" "B.Mask" "B.Paste") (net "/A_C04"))
  (pad "C05" smd circle (at 6.6675 0.79) (size 0.356 0.356) (layers "B.Cu" "B.Mask" "B.Paste") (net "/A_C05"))
  (pad "C06" smd circle (at 6.0325 0.79) (size 0.356 0.356) (layers "B.Cu" "B.Mask" "B.Paste") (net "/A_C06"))
  (pad "C07" smd circle (at 5.3975 0.79) (size 0.356 0.356) (layers "B.Cu" "B.Mask" "B.Paste") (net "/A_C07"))
  (pad "C08" smd circle (at 4.7625 0.79) (size 0.356 0.356) (layers "B.Cu" "B.Mask" "B.Paste") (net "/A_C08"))
  (pad "C09" smd circle (at 4.1275 0.79) (size 0.356 0.356) (layers "B.Cu" "B.Mask" "B.Paste") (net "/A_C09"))
  (pad "C10" smd circle (at 3.4925 0.79) (size 0.356 0.356) (layers "B.Cu" "B.Mask" "B.Paste") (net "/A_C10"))
  (pad "C11" smd circle (at 2.8575 0.79) (size 0.356 0.356) (layers "B.Cu" "B.Mask" "B.Paste") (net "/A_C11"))
  (pad "C12" smd circle (at 2.2225 0.79) (size 0.356 0.356) (layers "B.Cu" "B.Mask" "B.Paste") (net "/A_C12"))
  (pad "C13" smd circle (at 1.5875 0.79) (size 0.356 0.356) (layers "B.Cu" "B.Mask" "B.Paste") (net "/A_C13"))
  (pad "C14" smd circle (at 0.9525 0.79) (size 0.356 0.356) (layers "B.Cu" "B.Mask" "B.Paste") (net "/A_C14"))
  (pad "C15" smd circle (at 0.3175 0.79) (size 0.356 0.356) (layers "B.Cu" "B.Mask" "B.Paste") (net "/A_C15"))
  (pad "C16" smd circle (at -0.3175 0.79) (size 0.356 0.356) (layers "B.Cu" "B.Mask" "B.Paste") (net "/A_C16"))
  (pad "C17" smd circle (at -0.9525 0.79) (size 0.356 0.356) (layers "B.Cu" "B.Mask" "B.Paste") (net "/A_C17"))
  (pad "C18" smd circle (at -1.5875 0.79) (size 0.356 0.356) (layers "B.Cu" "B.Mask" "B.Paste") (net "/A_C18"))
  (pad "C19" smd circle (at -2.2225 0.79) (size 0.356 0.356) (layers "B.Cu" "B.Mask" "B.Paste") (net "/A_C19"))
  (pad "C20" smd circle (at -2.8575 0.79) (size 0.356 0.356) (layers "B.Cu" "B.Mask" "B.Paste") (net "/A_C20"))
  (pad "C21" smd circle (at -3.4925 0.79) (size 0.356 0.356) (layers "B.Cu" "B.Mask" "B.Paste") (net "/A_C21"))
  (pad "C22" smd circle (at -4.1275 0.79) (size 0.356 0.356) (layers "B.Cu" "B.Mask" "B.Paste") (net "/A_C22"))
  (pad "C23" smd circle (at -4.762499 0.79) (size 0.356 0.356) (layers "B.Cu" "B.Mask" "B.Paste") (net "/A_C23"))
  (pad "C24" smd circle (at -5.3975 0.79) (size 0.356 0.356) (layers "B.Cu" "B.Mask" "B.Paste") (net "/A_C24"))
  (pad "C25" smd circle (at -6.0325 0.79) (size 0.356 0.356) (layers "B.Cu" "B.Mask" "B.Paste") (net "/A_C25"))
  (pad "C26" smd circle (at -6.667499 0.79) (size 0.356 0.356) (layers "B.Cu" "B.Mask" "B.Paste") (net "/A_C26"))
  (pad "C27" smd circle (at -7.3025 0.79) (size 0.356 0.356) (layers "B.Cu" "B.Mask" "B.Paste") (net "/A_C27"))
  (pad "C28" smd circle (at -7.9375 0.79) (size 0.356 0.356) (layers "B.Cu" "B.Mask" "B.Paste") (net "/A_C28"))
  (pad "C29" smd circle (at -8.572499 0.79) (size 0.356 0.356) (layers "B.Cu" "B.Mask" "B.Paste") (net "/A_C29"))
  (pad "C30" smd circle (at -9.2075 0.79) (size 0.356 0.356) (layers "B.Cu" "B.Mask" "B.Paste") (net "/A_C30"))
  (pad "D01" smd circle (at 9.2075 1.75) (size 0.356 0.356) (layers "B.Cu" "B.Mask" "B.Paste") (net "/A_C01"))
  (pad "D02" smd circle (at 8.5725 1.75) (size 0.356 0.356) (layers "B.Cu" "B.Mask" "B.Paste") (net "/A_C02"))
  (pad "D03" smd circle (at 7.9375 1.75) (size 0.356 0.356) (layers "B.Cu" "B.Mask" "B.Paste") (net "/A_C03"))
  (pad "D04" smd circle (at 7.3025 1.75) (size 0.356 0.356) (layers "B.Cu" "B.Mask" "B.Paste") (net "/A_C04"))
  (pad "D05" smd circle (at 6.6675 1.75) (size 0.356 0.356) (layers "B.Cu" "B.Mask" "B.Paste") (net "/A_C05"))
  (pad "D06" smd circle (at 6.0325 1.75) (size 0.356 0.356) (layers "B.Cu" "B.Mask" "B.Paste") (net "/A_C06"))
  (pad "D07" smd circle (at 5.3975 1.75) (size 0.356 0.356) (layers "B.Cu" "B.Mask" "B.Paste") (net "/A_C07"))
  (pad "D08" smd circle (at 4.7625 1.75) (size 0.356 0.356) (layers "B.Cu" "B.Mask" "B.Paste") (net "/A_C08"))
  (pad "D09" smd circle (at 4.1275 1.75) (size 0.356 0.356) (layers "B.Cu" "B.Mask" "B.Paste") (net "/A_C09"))
  (pad "D10" smd circle (at 3.4925 1.75) (size 0.356 0.356) (layers "B.Cu" "B.Mask" "B.Paste") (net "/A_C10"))
  (pad "D11" smd circle (at 2.8575 1.75) (size 0.356 0.356) (layers "B.Cu" "B.Mask" "B.Paste") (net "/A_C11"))
  (pad "D12" smd circle (at 2.2225 1.75) (size 0.356 0.356) (layers "B.Cu" "B.Mask" "B.Paste") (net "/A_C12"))
  (pad "D13" smd circle (at 1.5875 1.75) (size 0.356 0.356) (layers "B.Cu" "B.Mask" "B.Paste") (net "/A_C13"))
  (pad "D14" smd circle (at 0.9525 1.75) (size 0.356 0.356) (layers "B.Cu" "B.Mask" "B.Paste") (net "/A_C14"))
  (pad "D15" smd circle (at 0.3175 1.75) (size 0.356 0.356) (layers "B.Cu" "B.Mask" "B.Paste") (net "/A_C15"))
  (pad "D16" smd circle (at -0.3175 1.75) (size 0.356 0.356) (layers "B.Cu" "B.Mask" "B.Paste") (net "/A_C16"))
  (pad "D17" smd circle (at -0.9525 1.75) (size 0.356 0.356) (layers "B.Cu" "B.Mask" "B.Paste") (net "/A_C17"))
  (pad "D18" smd circle (at -1.5875 1.75) (size 0.356 0.356) (layers "B.Cu" "B.Mask" "B.Paste") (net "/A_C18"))
  (pad "D19" smd circle (at -2.2225 1.75) (size 0.356 0.356) (layers "B.Cu" "B.Mask" "B.Paste") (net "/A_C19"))
  (pad "D20" smd circle (at -2.8575 1.75) (size 0.356 0.356) (layers "B.Cu" "B.Mask" "B.Paste") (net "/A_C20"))
  (pad "D21" smd circle (at -3.4925 1.75) (size 0.356 0.356) (layers "B.Cu" "B.Mask" "B.Paste") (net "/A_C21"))
  (pad "D22" smd circle (at -4.1275 1.75) (size 0.356 0.356) (layers "B.Cu" "B.Mask" "B.Paste") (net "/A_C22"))
  (pad "D23" smd circle (at -4.762499 1.75) (size 0.356 0.356) (layers "B.Cu" "B.Mask" "B.Paste") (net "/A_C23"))
  (pad "D24" smd circle (at -5.3975 1.75) (size 0.356 0.356) (layers "B.Cu" "B.Mask" "B.Paste") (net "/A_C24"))
  (pad "D25" smd circle (at -6.0325 1.75) (size 0.356 0.356) (layers "B.Cu" "B.Mask" "B.Paste") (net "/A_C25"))
  (pad "D26" smd circle (at -6.667499 1.75) (size 0.356 0.356) (layers "B.Cu" "B.Mask" "B.Paste") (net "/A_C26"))
  (pad "D27" smd circle (at -7.3025 1.75) (size 0.356 0.356) (layers "B.Cu" "B.Mask" "B.Paste") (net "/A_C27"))
  (pad "D28" smd circle (at -7.9375 1.75) (size 0.356 0.356) (layers "B.Cu" "B.Mask" "B.Paste") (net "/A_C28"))
  (pad "D29" smd circle (at -8.572499 1.75) (size 0.356 0.356) (layers "B.Cu" "B.Mask" "B.Paste") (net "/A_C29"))
  (pad "D30" smd circle (at -9.2075 1.75) (size 0.356 0.356) (layers "B.Cu" "B.Mask" "B.Paste") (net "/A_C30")))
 (gr_rect (start 100 100) (end 150 140) (stroke (width 0.1) (type solid)) (fill no) (layer "Edge.Cuts"))
 (segment (start 134.2075 103.25) (end 134.2075 104.21) (width 0.2) (layer "B.Cu") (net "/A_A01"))
 (segment (start 133.5725 103.25) (end 133.5725 104.21) (width 0.2) (layer "B.Cu") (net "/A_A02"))
 (segment (start 132.9375 103.25) (end 132.9375 104.21) (width 0.2) (layer "B.Cu") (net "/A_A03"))
 (segment (start 132.3025 103.25) (end 132.3025 104.21) (width 0.2) (layer "B.Cu") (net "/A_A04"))
 (segment (start 131.6675 103.25) (end 131.6675 104.21) (width 0.2) (layer "B.Cu") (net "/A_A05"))
 (segment (start 131.0325 103.25) (end 131.0325 104.21) (width 0.2) (layer "B.Cu") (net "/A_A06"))
 (segment (start 130.3975 103.25) (end 130.3975 104.21) (width 0.2) (layer "B.Cu") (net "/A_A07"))
 (segment (start 129.7625 103.25) (end 129.7625 104.21) (width 0.2) (layer "B.Cu") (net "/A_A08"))
 (segment (start 129.1275 103.25) (end 129.1275 104.21) (width 0.2) (layer "B.Cu") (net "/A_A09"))
 (segment (start 128.4925 103.25) (end 128.4925 104.21) (width 0.2) (layer "B.Cu") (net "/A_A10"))
 (segment (start 127.8575 103.25) (end 127.8575 104.21) (width 0.2) (layer "B.Cu") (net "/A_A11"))
 (segment (start 127.2225 103.25) (end 127.2225 104.21) (width 0.2) (layer "B.Cu") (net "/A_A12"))
 (segment (start 126.5875 103.25) (end 126.5875 104.21) (width 0.2) (layer "B.Cu") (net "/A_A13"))
 (segment (start 125.9525 103.25) (end 125.9525 104.21) (width 0.2) (layer "B.Cu") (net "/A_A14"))
 (segment (start 125.3175 103.25) (end 125.3175 104.21) (width 0.2) (layer "B.Cu") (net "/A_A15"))
 (segment (start 124.6825 103.25) (end 124.6825 104.21) (width 0.2) (layer "B.Cu") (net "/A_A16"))
 (segment (start 124.0475 103.25) (end 124.0475 104.21) (width 0.2) (layer "B.Cu") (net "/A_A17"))
 (segment (start 123.4125 103.25) (end 123.4125 104.21) (width 0.2) (layer "B.Cu") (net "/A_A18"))
 (segment (start 122.7775 103.25) (end 122.7775 104.21) (width 0.2) (layer "B.Cu") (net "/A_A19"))
 (segment (start 122.1425 103.25) (end 122.1425 104.21) (width 0.2) (layer "B.Cu") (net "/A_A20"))
 (segment (start 121.5075 103.25) (end 121.5075 104.21) (width 0.2) (layer "B.Cu") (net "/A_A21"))
 (segment (start 120.8725 103.25) (end 120.8725 104.21) (width 0.2) (layer "B.Cu") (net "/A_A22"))
 (segment (start 120.237501 103.25) (end 120.237501 104.21) (width 0.2) (layer "B.Cu") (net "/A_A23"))
 (segment (start 119.6025 103.25) (end 119.6025 104.21) (width 0.2) (layer "B.Cu") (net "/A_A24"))
 (segment (start 118.9675 103.25) (end 118.9675 104.21) (width 0.2) (layer "B.Cu") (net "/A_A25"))
 (segment (start 118.332501 103.25) (end 118.332501 104.21) (width 0.2) (layer "B.Cu") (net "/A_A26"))
 (segment (start 117.6975 103.25) (end 117.6975 104.21) (width 0.2) (layer "B.Cu") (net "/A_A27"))
 (segment (start 117.0625 103.25) (end 117.0625 104.21) (width 0.2) (layer "B.Cu") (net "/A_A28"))
 (segment (start 116.427501 103.25) (end 116.427501 104.21) (width 0.2) (layer "B.Cu") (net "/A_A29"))
 (segment (start 115.7925 103.25) (end 115.7925 104.21) (width 0.2) (layer "B.Cu") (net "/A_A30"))
 (segment (start 134.2075 105.79) (end 134.2075 106.75) (width 0.2) (layer "B.Cu") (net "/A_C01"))
 (segment (start 133.5725 105.79) (end 133.5725 106.75) (width 0.2) (layer "B.Cu") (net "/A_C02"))
 (segment (start 132.9375 105.79) (end 132.9375 106.75) (width 0.2) (layer "B.Cu") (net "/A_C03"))
 (segment (start 132.3025 105.79) (end 132.3025 106.75) (width 0.2) (layer "B.Cu") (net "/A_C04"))
 (segment (start 131.6675 105.79) (end 131.6675 106.75) (width 0.2) (layer "B.Cu") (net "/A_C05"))
 (segment (start 131.0325 105.79) (end 131.0325 106.75) (width 0.2) (layer "B.Cu") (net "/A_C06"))
 (segment (start 130.3975 105.79) (end 130.3975 106.75) (width 0.2) (layer "B.Cu") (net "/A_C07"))
 (segment (start 129.7625 105.79) (end 129.7625 106.75) (width 0.2) (layer "B.Cu") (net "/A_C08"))
 (segment (start 129.1275 105.79) (end 129.1275 106.75) (width 0.2) (layer "B.Cu") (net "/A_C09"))
 (segment (start 128.4925 105.79) (end 128.4925 106.75) (width 0.2) (layer "B.Cu") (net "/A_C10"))
 (segment (start 127.8575 105.79) (end 127.8575 106.75) (width 0.2) (layer "B.Cu") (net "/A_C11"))
 (segment (start 127.2225 105.79) (end 127.2225 106.75) (width 0.2) (layer "B.Cu") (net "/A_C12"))
 (segment (start 126.5875 105.79) (end 126.5875 106.75) (width 0.2) (layer "B.Cu") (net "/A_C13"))
 (segment (start 125.9525 105.79) (end 125.9525 106.75) (width 0.2) (layer "B.Cu") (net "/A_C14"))
 (segment (start 125.3175 105.79) (end 125.3175 106.75) (width 0.2) (layer "B.Cu") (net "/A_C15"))
 (segment (start 124.6825 105.79) (end 124.6825 106.75) (width 0.2) (layer "B.Cu") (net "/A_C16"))
 (segment (start 124.0475 105.79) (end 124.0475 106.75) (width 0.2) (layer "B.Cu") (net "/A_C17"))
 (segment (start 123.4125 105.79) (end 123.4125 106.75) (width 0.2) (layer "B.Cu") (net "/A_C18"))
 (segment (start 122.7775 105.79) (end 122.7775 106.75) (width 0.2) (layer "B.Cu") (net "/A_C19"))
 (segment (start 122.1425 105.79) (end 122.1425 106.75) (width 0.2) (layer "B.Cu") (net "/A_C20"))
 (segment (start 121.5075 105.79) (end 121.5075 106.75) (width 0.2) (layer "B.Cu") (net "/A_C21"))
 (segment (start 120.8725 105.79) (end 120.8725 106.75) (width 0.2) (layer "B.Cu") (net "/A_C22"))
 (segment (start 120.237501 105.79) (end 120.237501 106.75) (width 0.2) (layer "B.Cu") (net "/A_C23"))
 (segment (start 119.6025 105.79) (end 119.6025 106.75) (width 0.2) (layer "B.Cu") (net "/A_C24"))
 (segment (start 118.9675 105.79) (end 118.9675 106.75) (width 0.2) (layer "B.Cu") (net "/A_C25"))
 (segment (start 118.332501 105.79) (end 118.332501 106.75) (width 0.2) (layer "B.Cu") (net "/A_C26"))
 (segment (start 117.6975 105.79) (end 117.6975 106.75) (width 0.2) (layer "B.Cu") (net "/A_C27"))
 (segment (start 117.0625 105.79) (end 117.0625 106.75) (width 0.2) (layer "B.Cu") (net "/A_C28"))
 (segment (start 116.427501 105.79) (end 116.427501 106.75) (width 0.2) (layer "B.Cu") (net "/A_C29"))
 (segment (start 115.7925 105.79) (end 115.7925 106.75) (width 0.2) (layer "B.Cu") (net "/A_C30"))
 (segment (start 135.7075 133.25) (end 135.7075 134.21) (width 0.2) (layer "B.Cu") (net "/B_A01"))
 (segment (start 135.0725 133.25) (end 135.0725 134.21) (width 0.2) (layer "B.Cu") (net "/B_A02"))
 (segment (start 134.4375 133.25) (end 134.4375 134.21) (width 0.2) (layer "B.Cu") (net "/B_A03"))
 (segment (start 133.8025 133.25) (end 133.8025 134.21) (width 0.2) (layer "B.Cu") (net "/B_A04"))
 (segment (start 133.1675 133.25) (end 133.1675 134.21) (width 0.2) (layer "B.Cu") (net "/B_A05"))
 (segment (start 132.5325 133.25) (end 132.5325 134.21) (width 0.2) (layer "B.Cu") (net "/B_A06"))
 (segment (start 131.8975 133.25) (end 131.8975 134.21) (width 0.2) (layer "B.Cu") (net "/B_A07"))
 (segment (start 131.2625 133.25) (end 131.2625 134.21) (width 0.2) (layer "B.Cu") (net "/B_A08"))
 (segment (start 130.6275 133.25) (end 130.6275 134.21) (width 0.2) (layer "B.Cu") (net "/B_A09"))
 (segment (start 129.9925 133.25) (end 129.9925 134.21) (width 0.2) (layer "B.Cu") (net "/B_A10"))
 (segment (start 129.3575 133.25) (end 129.3575 134.21) (width 0.2) (layer "B.Cu") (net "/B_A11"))
 (segment (start 128.7225 133.25) (end 128.7225 134.21) (width 0.2) (layer "B.Cu") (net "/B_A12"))
 (segment (start 128.0875 133.25) (end 128.0875 134.21) (width 0.2) (layer "B.Cu") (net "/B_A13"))
 (segment (start 127.4525 133.25) (end 127.4525 134.21) (width 0.2) (layer "B.Cu") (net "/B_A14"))
 (segment (start 126.8175 133.25) (end 126.8175 134.21) (width 0.2) (layer "B.Cu") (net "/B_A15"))
 (segment (start 126.1825 133.25) (end 126.1825 134.21) (width 0.2) (layer "B.Cu") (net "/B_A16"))
 (segment (start 125.5475 133.25) (end 125.5475 134.21) (width 0.2) (layer "B.Cu") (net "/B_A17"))
 (segment (start 124.9125 133.25) (end 124.9125 134.21) (width 0.2) (layer "B.Cu") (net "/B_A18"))
 (segment (start 124.2775 133.25) (end 124.2775 134.21) (width 0.2) (layer "B.Cu") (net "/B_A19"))
 (segment (start 123.642501 133.25) (end 123.642501 134.21) (width 0.2) (layer "B.Cu") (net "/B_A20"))
 (segment (start 123.0075 133.25) (end 123.0075 134.21) (width 0.2) (layer "B.Cu") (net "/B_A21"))
 (segment (start 122.3725 133.25) (end 122.3725 134.21) (width 0.2) (layer "B.Cu") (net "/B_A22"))
 (segment (start 121.737501 133.25) (end 121.737501 134.21) (width 0.2) (layer "B.Cu") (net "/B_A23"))
 (segment (start 121.1025 133.25) (end 121.1025 134.21) (width 0.2) (layer "B.Cu") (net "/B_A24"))
 (segment (start 120.4675 133.25) (end 120.4675 134.21) (width 0.2) (layer "B.Cu") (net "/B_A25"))
 (segment (start 119.832501 133.25) (end 119.832501 134.21) (width 0.2) (layer "B.Cu") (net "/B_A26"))
 (segment (start 119.1975 133.25) (end 119.1975 134.21) (width 0.2) (layer "B.Cu") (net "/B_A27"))
 (segment (start 118.5625 133.25) (end 118.5625 134.21) (width 0.2) (layer "B.Cu") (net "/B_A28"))
 (segment (start 117.9275 133.25) (end 117.9275 134.21) (width 0.2) (layer "B.Cu") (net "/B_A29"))
 (segment (start 117.2925 133.25) (end 117.2925 134.21) (width 0.2) (layer "B.Cu") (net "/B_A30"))
 (segment (start 135.7075 135.79) (end 135.7075 136.75) (width 0.2) (layer "B.Cu") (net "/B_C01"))
 (segment (start 135.0725 135.79) (end 135.0725 136.75) (width 0.2) (layer "B.Cu") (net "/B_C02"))
 (segment (start 134.4375 135.79) (end 134.4375 136.75) (width 0.2) (layer "B.Cu") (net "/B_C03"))
 (segment (start 133.8025 135.79) (end 133.8025 136.75) (width 0.2) (layer "B.Cu") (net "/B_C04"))
 (segment (start 133.1675 135.79) (end 133.1675 136.75) (width 0.2) (layer "B.Cu") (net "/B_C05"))
 (segment (start 132.5325 135.79) (end 132.5325 136.75) (width 0.2) (layer "B.Cu") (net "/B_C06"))
 (segment (start 131.8975 135.79) (end 131.8975 136.75) (width 0.2) (layer "B.Cu") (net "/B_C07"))
 (segment (start 131.2625 135.79) (end 131.2625 136.75) (width 0.2) (layer "B.Cu") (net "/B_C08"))
 (segment (start 130.6275 135.79) (end 130.6275 136.75) (width 0.2) (layer "B.Cu") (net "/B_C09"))
 (segment (start 129.9925 135.79) (end 129.9925 136.75) (width 0.2) (layer "B.Cu") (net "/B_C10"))
 (segment (start 129.3575 135.79) (end 129.3575 136.75) (width 0.2) (layer "B.Cu") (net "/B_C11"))
 (segment (start 128.7225 135.79) (end 128.7225 136.75) (width 0.2) (layer "B.Cu") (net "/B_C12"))
 (segment (start 128.0875 135.79) (end 128.0875 136.75) (width 0.2) (layer "B.Cu") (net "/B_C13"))
 (segment (start 127.4525 135.79) (end 127.4525 136.75) (width 0.2) (layer "B.Cu") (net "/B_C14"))
 (segment (start 126.8175 135.79) (end 126.8175 136.75) (width 0.2) (layer "B.Cu") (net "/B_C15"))
 (segment (start 126.1825 135.79) (end 126.1825 136.75) (width 0.2) (layer "B.Cu") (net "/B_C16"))
 (segment (start 125.5475 135.79) (end 125.5475 136.75) (width 0.2) (layer "B.Cu") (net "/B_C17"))
 (segment (start 124.9125 135.79) (end 124.9125 136.75) (width 0.2) (layer "B.Cu") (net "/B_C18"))
 (segment (start 124.2775 135.79) (end 124.2775 136.75) (width 0.2) (layer "B.Cu") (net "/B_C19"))
 (segment (start 123.642501 135.79) (end 123.642501 136.75) (width 0.2) (layer "B.Cu") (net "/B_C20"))
 (segment (start 123.0075 135.79) (end 123.0075 136.75) (width 0.2) (layer "B.Cu") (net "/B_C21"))
 (segment (start 122.3725 135.79) (end 122.3725 136.75) (width 0.2) (layer "B.Cu") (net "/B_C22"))
 (segment (start 121.737501 135.79) (end 121.737501 136.75) (width 0.2) (layer "B.Cu") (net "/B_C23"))
 (segment (start 121.1025 135.79) (end 121.1025 136.75) (width 0.2) (layer "B.Cu") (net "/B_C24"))
 (segment (start 120.4675 135.79) (end 120.4675 136.75) (width 0.2) (layer "B.Cu") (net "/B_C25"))
 (segment (start 119.832501 135.79) (end 119.832501 136.75) (width 0.2) (layer "B.Cu") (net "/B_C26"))
 (segment (start 119.1975 135.79) (end 119.1975 136.75) (width 0.2) (layer "B.Cu") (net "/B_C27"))
 (segment (start 118.5625 135.79) (end 118.5625 136.75) (width 0.2) (layer "B.Cu") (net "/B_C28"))
 (segment (start 117.9275 135.79) (end 117.9275 136.75) (width 0.2) (layer "B.Cu") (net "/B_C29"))
 (segment (start 117.2925 135.79) (end 117.2925 136.75) (width 0.2) (layer "B.Cu") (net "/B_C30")))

